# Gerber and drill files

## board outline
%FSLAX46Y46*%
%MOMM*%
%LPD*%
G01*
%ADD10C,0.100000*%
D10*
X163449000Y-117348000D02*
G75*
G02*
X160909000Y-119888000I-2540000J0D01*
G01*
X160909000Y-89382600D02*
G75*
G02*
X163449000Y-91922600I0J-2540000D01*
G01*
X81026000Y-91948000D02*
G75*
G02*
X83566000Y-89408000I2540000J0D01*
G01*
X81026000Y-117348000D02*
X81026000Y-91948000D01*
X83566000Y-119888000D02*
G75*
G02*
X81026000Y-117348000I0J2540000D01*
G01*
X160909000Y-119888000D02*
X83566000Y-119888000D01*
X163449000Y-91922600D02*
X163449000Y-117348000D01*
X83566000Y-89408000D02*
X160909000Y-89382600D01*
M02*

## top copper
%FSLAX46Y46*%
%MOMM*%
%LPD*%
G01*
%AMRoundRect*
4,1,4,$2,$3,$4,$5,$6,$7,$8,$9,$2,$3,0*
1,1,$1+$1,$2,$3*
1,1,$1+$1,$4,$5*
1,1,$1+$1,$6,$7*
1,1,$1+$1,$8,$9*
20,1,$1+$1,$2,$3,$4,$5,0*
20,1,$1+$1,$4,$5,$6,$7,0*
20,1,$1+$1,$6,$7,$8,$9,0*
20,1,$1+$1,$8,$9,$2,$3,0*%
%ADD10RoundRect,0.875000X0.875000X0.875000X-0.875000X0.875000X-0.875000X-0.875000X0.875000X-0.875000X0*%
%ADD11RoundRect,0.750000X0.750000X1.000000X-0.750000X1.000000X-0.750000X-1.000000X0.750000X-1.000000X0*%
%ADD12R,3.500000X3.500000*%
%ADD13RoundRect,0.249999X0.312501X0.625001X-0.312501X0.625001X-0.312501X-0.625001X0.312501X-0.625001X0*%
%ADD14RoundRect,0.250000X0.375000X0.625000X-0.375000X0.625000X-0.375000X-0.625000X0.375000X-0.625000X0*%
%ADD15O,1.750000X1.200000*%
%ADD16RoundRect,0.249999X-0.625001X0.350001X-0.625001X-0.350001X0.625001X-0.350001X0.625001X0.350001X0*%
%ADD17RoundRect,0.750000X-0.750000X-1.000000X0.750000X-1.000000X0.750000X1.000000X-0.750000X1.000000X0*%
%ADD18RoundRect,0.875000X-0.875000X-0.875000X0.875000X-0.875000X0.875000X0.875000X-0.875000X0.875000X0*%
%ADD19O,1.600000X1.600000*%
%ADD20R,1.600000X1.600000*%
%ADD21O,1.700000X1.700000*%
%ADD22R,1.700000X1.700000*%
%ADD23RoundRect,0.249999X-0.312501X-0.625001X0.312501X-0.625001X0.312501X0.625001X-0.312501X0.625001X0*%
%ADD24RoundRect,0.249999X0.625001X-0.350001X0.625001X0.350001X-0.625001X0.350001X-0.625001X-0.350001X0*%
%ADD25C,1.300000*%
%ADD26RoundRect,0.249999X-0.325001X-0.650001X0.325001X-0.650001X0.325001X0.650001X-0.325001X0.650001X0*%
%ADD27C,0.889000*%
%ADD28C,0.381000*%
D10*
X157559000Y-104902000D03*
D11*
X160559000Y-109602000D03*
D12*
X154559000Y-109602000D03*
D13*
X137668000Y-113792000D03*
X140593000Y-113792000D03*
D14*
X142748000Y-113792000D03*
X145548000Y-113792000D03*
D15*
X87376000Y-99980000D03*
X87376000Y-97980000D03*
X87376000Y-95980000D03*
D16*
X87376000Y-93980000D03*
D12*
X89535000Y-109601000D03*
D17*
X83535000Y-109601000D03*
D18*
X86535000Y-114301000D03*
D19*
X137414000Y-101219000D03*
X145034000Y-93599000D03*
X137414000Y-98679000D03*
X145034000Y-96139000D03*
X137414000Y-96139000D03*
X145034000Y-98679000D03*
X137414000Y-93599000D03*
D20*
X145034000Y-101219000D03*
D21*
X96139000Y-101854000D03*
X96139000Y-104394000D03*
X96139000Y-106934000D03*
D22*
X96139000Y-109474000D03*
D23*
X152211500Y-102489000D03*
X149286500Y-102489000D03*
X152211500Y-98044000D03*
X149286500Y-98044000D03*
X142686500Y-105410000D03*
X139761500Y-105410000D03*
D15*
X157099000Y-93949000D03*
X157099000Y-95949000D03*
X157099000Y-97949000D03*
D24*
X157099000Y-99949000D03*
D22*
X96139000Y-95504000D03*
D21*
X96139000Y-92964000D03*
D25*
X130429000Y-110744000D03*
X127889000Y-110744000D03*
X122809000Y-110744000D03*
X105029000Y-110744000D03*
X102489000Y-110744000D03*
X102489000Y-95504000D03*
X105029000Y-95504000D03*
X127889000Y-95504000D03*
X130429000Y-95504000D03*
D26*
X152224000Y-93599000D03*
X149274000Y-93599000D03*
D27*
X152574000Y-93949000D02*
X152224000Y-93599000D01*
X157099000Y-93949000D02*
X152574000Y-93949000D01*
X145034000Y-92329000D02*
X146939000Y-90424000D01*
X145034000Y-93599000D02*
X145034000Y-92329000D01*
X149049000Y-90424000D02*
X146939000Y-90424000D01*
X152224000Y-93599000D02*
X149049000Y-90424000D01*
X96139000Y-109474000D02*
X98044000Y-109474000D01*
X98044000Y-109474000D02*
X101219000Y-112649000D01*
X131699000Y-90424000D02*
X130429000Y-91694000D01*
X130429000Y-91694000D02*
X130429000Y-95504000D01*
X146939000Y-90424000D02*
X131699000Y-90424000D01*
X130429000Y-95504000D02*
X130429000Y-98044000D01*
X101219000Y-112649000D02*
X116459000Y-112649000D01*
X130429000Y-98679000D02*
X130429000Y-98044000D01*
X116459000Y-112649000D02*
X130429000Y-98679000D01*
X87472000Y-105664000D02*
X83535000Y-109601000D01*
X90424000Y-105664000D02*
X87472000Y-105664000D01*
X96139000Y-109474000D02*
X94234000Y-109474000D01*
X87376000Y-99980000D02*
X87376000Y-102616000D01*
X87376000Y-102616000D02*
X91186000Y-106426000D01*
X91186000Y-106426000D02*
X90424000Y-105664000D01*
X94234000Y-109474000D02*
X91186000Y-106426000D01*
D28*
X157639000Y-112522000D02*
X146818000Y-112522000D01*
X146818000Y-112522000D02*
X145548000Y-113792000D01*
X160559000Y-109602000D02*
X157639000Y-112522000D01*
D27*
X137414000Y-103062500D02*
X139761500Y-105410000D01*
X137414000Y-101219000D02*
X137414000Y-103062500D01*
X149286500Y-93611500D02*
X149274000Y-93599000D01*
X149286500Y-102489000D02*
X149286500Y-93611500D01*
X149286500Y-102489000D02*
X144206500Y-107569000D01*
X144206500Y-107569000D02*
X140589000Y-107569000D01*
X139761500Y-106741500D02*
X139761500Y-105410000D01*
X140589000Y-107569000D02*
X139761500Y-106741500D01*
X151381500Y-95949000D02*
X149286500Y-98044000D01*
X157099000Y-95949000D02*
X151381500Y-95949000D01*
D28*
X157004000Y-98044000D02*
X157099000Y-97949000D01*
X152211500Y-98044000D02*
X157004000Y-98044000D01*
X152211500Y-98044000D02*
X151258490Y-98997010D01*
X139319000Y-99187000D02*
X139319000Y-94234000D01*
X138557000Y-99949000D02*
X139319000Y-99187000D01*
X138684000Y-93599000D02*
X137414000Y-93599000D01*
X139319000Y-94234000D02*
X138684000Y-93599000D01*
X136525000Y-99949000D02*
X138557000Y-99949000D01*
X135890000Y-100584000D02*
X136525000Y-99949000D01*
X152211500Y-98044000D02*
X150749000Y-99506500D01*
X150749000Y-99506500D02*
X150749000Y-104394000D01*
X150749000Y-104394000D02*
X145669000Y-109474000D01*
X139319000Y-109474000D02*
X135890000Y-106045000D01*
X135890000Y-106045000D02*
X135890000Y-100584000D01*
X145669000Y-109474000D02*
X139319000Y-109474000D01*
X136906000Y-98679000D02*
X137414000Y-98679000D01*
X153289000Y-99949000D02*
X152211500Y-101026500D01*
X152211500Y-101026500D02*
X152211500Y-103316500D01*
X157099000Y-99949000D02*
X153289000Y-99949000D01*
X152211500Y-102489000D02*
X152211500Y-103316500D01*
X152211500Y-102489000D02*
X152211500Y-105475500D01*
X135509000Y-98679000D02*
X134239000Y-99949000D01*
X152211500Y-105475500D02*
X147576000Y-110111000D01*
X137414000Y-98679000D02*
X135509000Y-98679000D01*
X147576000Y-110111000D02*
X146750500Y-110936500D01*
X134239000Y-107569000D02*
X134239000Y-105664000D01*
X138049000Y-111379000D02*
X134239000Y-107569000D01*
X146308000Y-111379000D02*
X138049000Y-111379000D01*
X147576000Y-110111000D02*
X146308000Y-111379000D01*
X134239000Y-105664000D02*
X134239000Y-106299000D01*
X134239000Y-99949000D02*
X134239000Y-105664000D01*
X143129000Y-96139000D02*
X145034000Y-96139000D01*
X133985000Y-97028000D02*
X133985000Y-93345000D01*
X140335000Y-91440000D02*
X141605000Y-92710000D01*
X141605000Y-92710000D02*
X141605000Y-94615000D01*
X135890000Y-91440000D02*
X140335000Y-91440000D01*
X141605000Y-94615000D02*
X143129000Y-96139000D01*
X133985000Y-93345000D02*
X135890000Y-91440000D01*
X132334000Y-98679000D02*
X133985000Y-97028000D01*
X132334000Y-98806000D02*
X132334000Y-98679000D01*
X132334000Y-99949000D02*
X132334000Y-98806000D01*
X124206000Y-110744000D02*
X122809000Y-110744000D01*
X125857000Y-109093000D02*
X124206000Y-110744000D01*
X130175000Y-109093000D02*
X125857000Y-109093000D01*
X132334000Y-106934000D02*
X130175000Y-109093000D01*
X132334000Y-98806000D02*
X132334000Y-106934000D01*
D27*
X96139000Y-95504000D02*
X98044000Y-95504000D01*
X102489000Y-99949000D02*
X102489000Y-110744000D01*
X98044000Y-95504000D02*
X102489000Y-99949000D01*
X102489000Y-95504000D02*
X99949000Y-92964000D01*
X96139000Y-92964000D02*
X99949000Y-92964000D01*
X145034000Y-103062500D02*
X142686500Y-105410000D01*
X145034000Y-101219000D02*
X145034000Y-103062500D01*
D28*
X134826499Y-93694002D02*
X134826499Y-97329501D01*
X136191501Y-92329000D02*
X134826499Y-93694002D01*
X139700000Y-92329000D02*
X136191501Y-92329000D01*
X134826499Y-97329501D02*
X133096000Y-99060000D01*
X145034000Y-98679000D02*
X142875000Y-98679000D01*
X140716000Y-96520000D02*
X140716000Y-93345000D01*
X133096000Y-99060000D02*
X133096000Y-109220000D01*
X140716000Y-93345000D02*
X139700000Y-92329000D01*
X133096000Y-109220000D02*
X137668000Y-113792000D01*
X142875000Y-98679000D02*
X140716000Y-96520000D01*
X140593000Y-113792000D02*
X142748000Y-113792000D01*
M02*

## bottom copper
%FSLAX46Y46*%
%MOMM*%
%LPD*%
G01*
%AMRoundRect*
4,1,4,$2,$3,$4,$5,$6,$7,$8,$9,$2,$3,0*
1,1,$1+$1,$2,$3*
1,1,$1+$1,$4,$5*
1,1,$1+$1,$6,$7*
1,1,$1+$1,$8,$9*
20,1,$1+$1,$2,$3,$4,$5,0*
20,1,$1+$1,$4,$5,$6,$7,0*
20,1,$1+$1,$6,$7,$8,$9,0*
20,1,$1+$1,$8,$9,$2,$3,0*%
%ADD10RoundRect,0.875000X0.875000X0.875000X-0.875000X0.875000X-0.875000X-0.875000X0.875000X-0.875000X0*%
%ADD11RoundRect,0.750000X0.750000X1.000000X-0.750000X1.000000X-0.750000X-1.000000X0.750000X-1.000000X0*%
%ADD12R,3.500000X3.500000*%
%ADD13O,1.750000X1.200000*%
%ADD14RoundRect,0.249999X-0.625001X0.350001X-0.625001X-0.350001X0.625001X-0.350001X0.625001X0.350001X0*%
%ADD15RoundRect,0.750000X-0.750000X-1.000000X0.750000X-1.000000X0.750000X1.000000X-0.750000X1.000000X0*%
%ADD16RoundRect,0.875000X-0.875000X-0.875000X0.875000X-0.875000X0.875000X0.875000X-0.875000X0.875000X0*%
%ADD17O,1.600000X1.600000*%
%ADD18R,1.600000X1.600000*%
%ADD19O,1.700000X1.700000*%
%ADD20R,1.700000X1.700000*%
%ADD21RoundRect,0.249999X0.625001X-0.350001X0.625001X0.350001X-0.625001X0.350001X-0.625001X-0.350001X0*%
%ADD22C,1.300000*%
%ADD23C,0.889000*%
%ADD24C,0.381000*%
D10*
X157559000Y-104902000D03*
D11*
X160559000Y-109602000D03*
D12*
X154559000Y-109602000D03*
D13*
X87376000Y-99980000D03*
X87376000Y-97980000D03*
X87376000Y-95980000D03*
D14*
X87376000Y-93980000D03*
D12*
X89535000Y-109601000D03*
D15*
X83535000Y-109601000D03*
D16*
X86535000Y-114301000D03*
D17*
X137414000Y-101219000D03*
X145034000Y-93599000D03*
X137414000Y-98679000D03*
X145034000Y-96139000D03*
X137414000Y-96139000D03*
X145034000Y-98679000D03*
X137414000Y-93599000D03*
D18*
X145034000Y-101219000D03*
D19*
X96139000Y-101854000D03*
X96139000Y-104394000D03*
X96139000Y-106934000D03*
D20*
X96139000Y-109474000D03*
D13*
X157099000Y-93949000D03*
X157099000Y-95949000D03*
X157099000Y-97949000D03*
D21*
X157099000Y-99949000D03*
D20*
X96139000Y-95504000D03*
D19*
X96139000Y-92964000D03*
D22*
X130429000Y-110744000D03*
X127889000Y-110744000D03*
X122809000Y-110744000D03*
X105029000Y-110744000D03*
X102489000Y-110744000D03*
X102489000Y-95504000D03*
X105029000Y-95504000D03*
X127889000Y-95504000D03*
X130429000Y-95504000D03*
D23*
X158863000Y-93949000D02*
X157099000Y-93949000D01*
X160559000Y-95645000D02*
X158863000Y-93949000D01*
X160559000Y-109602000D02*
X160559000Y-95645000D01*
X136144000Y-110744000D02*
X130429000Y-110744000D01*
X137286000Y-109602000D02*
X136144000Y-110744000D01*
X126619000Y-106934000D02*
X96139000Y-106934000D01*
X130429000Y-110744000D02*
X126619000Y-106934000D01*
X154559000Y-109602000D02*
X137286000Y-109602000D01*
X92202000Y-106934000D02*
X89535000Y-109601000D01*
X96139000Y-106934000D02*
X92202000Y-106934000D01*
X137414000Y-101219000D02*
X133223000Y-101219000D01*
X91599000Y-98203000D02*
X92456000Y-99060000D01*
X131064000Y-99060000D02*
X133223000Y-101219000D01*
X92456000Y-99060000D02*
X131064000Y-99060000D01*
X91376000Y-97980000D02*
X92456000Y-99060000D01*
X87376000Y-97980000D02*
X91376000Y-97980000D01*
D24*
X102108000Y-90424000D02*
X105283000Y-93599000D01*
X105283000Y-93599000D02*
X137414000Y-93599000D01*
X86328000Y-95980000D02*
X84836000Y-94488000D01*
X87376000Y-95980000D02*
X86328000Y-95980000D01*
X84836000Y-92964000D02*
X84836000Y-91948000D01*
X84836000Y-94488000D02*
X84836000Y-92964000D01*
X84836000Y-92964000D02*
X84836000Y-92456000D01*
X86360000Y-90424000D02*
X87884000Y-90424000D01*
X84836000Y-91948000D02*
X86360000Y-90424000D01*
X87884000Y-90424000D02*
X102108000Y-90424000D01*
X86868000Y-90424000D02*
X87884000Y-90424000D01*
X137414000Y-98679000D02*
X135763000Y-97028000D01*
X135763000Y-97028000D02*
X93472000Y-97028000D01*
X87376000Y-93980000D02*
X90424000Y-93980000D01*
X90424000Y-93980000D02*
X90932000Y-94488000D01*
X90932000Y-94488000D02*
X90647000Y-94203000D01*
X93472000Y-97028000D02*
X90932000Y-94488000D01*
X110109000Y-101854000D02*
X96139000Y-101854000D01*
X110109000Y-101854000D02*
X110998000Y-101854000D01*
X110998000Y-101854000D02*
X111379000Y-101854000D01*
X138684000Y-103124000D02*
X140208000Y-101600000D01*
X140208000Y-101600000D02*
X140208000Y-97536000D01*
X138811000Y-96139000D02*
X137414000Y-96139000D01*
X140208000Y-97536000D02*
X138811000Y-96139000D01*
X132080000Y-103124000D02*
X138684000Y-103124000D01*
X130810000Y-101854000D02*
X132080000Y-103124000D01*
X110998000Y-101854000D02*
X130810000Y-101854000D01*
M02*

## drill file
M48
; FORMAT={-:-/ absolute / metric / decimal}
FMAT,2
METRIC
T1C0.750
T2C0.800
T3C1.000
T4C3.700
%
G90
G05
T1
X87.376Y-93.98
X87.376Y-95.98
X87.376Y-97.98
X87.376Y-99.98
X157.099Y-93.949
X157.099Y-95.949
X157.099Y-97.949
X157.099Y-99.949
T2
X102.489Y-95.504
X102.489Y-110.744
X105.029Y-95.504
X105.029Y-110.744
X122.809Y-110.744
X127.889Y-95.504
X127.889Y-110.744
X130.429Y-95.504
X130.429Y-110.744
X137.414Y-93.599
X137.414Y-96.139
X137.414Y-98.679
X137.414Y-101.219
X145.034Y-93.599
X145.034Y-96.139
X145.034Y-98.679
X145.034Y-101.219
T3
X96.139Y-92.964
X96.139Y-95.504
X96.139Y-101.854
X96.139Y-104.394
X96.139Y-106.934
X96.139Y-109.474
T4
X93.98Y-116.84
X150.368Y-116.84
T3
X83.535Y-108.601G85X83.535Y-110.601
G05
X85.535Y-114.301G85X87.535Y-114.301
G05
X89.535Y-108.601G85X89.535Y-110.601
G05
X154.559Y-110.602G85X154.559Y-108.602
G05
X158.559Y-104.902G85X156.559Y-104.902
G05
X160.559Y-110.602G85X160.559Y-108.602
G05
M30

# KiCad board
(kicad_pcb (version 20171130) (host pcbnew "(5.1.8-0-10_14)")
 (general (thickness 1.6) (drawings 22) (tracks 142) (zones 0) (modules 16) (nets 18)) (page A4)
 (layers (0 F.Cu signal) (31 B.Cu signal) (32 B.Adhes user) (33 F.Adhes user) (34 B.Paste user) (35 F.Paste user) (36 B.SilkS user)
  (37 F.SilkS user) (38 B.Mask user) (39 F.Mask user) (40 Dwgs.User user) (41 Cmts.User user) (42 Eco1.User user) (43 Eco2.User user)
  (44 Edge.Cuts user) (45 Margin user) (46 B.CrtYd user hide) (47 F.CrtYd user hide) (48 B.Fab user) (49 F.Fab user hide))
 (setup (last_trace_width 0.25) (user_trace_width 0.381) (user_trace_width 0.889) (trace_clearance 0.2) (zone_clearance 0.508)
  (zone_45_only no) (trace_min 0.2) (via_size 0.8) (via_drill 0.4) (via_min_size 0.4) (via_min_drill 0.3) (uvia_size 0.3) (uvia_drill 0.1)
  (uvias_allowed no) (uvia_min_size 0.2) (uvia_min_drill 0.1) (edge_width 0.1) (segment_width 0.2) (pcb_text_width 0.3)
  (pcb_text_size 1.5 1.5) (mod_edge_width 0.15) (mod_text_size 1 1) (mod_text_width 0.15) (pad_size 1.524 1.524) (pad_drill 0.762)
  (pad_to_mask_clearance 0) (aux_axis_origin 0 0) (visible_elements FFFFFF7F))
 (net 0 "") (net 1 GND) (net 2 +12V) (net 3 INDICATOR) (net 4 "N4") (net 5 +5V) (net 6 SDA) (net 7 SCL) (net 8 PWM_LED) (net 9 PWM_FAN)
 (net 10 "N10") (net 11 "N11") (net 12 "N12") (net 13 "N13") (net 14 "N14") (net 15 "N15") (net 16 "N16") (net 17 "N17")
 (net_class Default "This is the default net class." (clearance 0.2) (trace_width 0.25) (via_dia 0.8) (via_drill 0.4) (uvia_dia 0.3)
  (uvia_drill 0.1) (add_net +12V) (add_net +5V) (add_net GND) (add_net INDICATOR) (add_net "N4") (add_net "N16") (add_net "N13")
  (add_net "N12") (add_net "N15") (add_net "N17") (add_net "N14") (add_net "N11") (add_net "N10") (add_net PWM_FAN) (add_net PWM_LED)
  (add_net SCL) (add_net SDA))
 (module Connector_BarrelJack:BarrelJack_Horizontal (layer F.Cu) (at 154.559 109.602 180)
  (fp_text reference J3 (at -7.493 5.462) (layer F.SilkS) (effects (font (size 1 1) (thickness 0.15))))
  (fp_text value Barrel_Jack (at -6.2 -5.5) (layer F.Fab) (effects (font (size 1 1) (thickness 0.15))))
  (pad 3 thru_hole roundrect (at -3 4.7 180) (size 3.5 3.5) (drill oval 3 1) (layers *.Cu *.Mask) (roundrect_rratio 0.25))
  (pad 2 thru_hole roundrect (at -6 0 180) (size 3 3.5) (drill oval 1 3) (layers *.Cu *.Mask) (roundrect_rratio 0.25) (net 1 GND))
  (pad 1 thru_hole rect (at 0 0 180) (size 3.5 3.5) (drill oval 1 3) (layers *.Cu *.Mask) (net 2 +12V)))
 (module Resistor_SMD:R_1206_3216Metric (layer F.Cu) (at 139.1305 113.792 180)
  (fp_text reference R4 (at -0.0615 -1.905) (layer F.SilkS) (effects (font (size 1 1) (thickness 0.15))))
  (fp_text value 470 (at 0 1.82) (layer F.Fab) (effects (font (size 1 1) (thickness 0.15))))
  (pad 2 smd roundrect (at 1.4625 0 180) (size 1.125 1.75) (layers F.Cu F.Paste F.Mask) (roundrect_rratio 0.2222213333333333)
   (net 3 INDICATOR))
  (pad 1 smd roundrect (at -1.4625 0 180) (size 1.125 1.75) (layers F.Cu F.Paste F.Mask) (roundrect_rratio 0.2222213333333333) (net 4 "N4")))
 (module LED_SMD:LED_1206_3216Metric (layer F.Cu) (at 144.148 113.792 180)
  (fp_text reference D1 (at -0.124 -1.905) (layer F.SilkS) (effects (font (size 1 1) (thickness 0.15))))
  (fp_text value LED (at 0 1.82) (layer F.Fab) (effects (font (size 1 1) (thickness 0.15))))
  (pad 2 smd roundrect (at 1.4 0 180) (size 1.25 1.75) (layers F.Cu F.Paste F.Mask) (roundrect_rratio 0.2) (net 4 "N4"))
  (pad 1 smd roundrect (at -1.4 0 180) (size 1.25 1.75) (layers F.Cu F.Paste F.Mask) (roundrect_rratio 0.2) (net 1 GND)))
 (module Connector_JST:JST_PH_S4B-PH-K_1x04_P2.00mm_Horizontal (layer F.Cu) (at 87.376 93.98 270)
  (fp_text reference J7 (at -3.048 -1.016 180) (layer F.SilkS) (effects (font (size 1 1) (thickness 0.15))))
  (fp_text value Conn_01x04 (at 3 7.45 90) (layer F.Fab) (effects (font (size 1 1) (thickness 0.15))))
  (pad 4 thru_hole oval (at 6 0 270) (size 1.2 1.75) (drill 0.75) (layers *.Cu *.Mask) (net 1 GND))
  (pad 3 thru_hole oval (at 4 0 270) (size 1.2 1.75) (drill 0.75) (layers *.Cu *.Mask) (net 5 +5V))
  (pad 2 thru_hole oval (at 2 0 270) (size 1.2 1.75) (drill 0.75) (layers *.Cu *.Mask) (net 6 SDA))
  (pad 1 thru_hole roundrect (at 0 0 270) (size 1.2 1.75) (drill 0.75) (layers *.Cu *.Mask) (roundrect_rratio 0.2083325) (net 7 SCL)))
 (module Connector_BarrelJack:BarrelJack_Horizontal (layer F.Cu) (at 89.535 109.601)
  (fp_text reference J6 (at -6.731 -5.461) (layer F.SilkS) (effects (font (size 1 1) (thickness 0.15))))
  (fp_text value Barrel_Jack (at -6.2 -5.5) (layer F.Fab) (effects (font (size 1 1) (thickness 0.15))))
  (pad 1 thru_hole rect (at 0 0) (size 3.5 3.5) (drill oval 1 3) (layers *.Cu *.Mask) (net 2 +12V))
  (pad 2 thru_hole roundrect (at -6 0) (size 3 3.5) (drill oval 1 3) (layers *.Cu *.Mask) (roundrect_rratio 0.25) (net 1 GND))
  (pad 3 thru_hole roundrect (at -3 4.7) (size 3.5 3.5) (drill oval 3 1) (layers *.Cu *.Mask) (roundrect_rratio 0.25)))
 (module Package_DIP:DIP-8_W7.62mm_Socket (layer F.Cu) (at 145.034 101.219 180)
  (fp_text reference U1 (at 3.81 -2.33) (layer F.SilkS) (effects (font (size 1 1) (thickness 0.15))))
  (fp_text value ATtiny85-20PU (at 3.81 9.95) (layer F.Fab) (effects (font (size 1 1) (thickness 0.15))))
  (pad 8 thru_hole oval (at 7.62 0 180) (size 1.6 1.6) (drill 0.8) (layers *.Cu *.Mask) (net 5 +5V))
  (pad 4 thru_hole oval (at 0 7.62 180) (size 1.6 1.6) (drill 0.8) (layers *.Cu *.Mask) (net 1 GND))
  (pad 7 thru_hole oval (at 7.62 2.54 180) (size 1.6 1.6) (drill 0.8) (layers *.Cu *.Mask) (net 7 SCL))
  (pad 3 thru_hole oval (at 0 5.08 180) (size 1.6 1.6) (drill 0.8) (layers *.Cu *.Mask) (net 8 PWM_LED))
  (pad 6 thru_hole oval (at 7.62 5.08 180) (size 1.6 1.6) (drill 0.8) (layers *.Cu *.Mask) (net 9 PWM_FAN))
  (pad 2 thru_hole oval (at 0 2.54 180) (size 1.6 1.6) (drill 0.8) (layers *.Cu *.Mask) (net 3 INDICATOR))
  (pad 5 thru_hole oval (at 7.62 7.62 180) (size 1.6 1.6) (drill 0.8) (layers *.Cu *.Mask) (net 6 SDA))
  (pad 1 thru_hole rect (at 0 0 180) (size 1.6 1.6) (drill 0.8) (layers *.Cu *.Mask) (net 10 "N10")))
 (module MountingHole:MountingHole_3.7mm (layer F.Cu) (at 150.368 116.84 180)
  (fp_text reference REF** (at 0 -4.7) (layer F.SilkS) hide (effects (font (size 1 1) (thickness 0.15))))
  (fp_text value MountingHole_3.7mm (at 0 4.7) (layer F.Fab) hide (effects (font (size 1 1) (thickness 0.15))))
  (pad 1 np_thru_hole circle (at 0 0 180) (size 3.7 3.7) (drill 3.7) (layers *.Cu *.Mask)))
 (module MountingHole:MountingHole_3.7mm (layer F.Cu) (at 93.98 116.84 180)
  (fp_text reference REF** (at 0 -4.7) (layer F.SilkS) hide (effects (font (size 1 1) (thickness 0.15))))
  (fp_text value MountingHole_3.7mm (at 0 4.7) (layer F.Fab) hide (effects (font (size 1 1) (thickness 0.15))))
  (pad 1 np_thru_hole circle (at 0 0 180) (size 3.7 3.7) (drill 3.7) (layers *.Cu *.Mask)))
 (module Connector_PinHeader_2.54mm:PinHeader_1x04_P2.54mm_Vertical (layer F.Cu) (at 96.139 109.474 180)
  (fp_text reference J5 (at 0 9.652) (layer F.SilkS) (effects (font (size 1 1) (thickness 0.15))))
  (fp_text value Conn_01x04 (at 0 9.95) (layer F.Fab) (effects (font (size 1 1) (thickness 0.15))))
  (pad 4 thru_hole oval (at 0 7.62 180) (size 1.7 1.7) (drill 1) (layers *.Cu *.Mask) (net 9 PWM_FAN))
  (pad 3 thru_hole oval (at 0 5.08 180) (size 1.7 1.7) (drill 1) (layers *.Cu *.Mask) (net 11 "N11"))
  (pad 2 thru_hole oval (at 0 2.54 180) (size 1.7 1.7) (drill 1) (layers *.Cu *.Mask) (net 2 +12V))
  (pad 1 thru_hole rect (at 0 0 180) (size 1.7 1.7) (drill 1) (layers *.Cu *.Mask) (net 1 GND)))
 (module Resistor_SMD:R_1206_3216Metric (layer F.Cu) (at 150.749 102.489)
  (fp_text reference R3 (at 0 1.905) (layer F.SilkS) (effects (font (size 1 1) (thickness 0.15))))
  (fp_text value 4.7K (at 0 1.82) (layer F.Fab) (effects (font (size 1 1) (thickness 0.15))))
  (pad 2 smd roundrect (at 1.4625 0) (size 1.125 1.75) (layers F.Cu F.Paste F.Mask) (roundrect_rratio 0.2222213333333333) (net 7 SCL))
  (pad 1 smd roundrect (at -1.4625 0) (size 1.125 1.75) (layers F.Cu F.Paste F.Mask) (roundrect_rratio 0.2222213333333333) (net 5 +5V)))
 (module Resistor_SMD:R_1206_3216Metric (layer F.Cu) (at 150.749 98.044)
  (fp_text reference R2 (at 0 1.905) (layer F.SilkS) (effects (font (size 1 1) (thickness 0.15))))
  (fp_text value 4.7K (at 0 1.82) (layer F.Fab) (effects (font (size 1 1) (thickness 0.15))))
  (pad 2 smd roundrect (at 1.4625 0) (size 1.125 1.75) (layers F.Cu F.Paste F.Mask) (roundrect_rratio 0.2222213333333333) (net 6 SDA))
  (pad 1 smd roundrect (at -1.4625 0) (size 1.125 1.75) (layers F.Cu F.Paste F.Mask) (roundrect_rratio 0.2222213333333333) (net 5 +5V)))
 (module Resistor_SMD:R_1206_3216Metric (layer F.Cu) (at 141.224 105.41)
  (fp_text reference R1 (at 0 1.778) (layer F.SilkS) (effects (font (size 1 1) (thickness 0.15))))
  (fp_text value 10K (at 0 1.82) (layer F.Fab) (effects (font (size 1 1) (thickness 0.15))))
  (pad 2 smd roundrect (at 1.4625 0) (size 1.125 1.75) (layers F.Cu F.Paste F.Mask) (roundrect_rratio 0.2222213333333333) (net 10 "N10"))
  (pad 1 smd roundrect (at -1.4625 0) (size 1.125 1.75) (layers F.Cu F.Paste F.Mask) (roundrect_rratio 0.2222213333333333) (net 5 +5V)))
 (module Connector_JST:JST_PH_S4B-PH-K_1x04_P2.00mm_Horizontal (layer F.Cu) (at 157.099 99.949 90)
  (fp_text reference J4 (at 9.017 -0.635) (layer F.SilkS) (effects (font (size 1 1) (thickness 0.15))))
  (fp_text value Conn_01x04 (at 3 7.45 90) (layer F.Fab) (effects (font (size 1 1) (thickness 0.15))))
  (pad 4 thru_hole oval (at 6 0 90) (size 1.2 1.75) (drill 0.75) (layers *.Cu *.Mask) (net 1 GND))
  (pad 3 thru_hole oval (at 4 0 90) (size 1.2 1.75) (drill 0.75) (layers *.Cu *.Mask) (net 5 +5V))
  (pad 2 thru_hole oval (at 2 0 90) (size 1.2 1.75) (drill 0.75) (layers *.Cu *.Mask) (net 6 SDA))
  (pad 1 thru_hole roundrect (at 0 0 90) (size 1.2 1.75) (drill 0.75) (layers *.Cu *.Mask) (roundrect_rratio 0.2083325) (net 7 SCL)))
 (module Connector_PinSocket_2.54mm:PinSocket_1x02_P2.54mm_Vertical (layer F.Cu) (at 96.139 95.504 180)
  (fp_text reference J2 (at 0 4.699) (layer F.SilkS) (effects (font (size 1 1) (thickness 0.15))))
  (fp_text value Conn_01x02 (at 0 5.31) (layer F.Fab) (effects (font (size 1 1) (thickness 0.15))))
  (pad 1 thru_hole rect (at 0 0 180) (size 1.7 1.7) (drill 1) (layers *.Cu *.Mask) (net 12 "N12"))
  (pad 2 thru_hole oval (at 0 2.54 180) (size 1.7 1.7) (drill 1) (layers *.Cu *.Mask) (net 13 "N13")))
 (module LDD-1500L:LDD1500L (layer F.Cu) (at 130.429 95.504 270)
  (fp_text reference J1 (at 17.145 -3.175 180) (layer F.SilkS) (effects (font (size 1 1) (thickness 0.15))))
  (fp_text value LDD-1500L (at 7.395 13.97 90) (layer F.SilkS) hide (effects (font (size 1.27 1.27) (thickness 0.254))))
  (pad 24 thru_hole circle (at 15.24 0) (size 1.3 1.3) (drill 0.8) (layers *.Cu *.Mask F.SilkS) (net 2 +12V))
  (pad 23 thru_hole circle (at 15.24 2.54) (size 1.3 1.3) (drill 0.8) (layers *.Cu *.Mask F.SilkS) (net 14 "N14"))
  (pad 21 thru_hole circle (at 15.24 7.62) (size 1.3 1.3) (drill 0.8) (layers *.Cu *.Mask F.SilkS) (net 8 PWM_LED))
  (pad 14 thru_hole circle (at 15.24 25.4) (size 1.3 1.3) (drill 0.8) (layers *.Cu *.Mask F.SilkS) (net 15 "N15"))
  (pad 13 thru_hole circle (at 15.24 27.94) (size 1.3 1.3) (drill 0.8) (layers *.Cu *.Mask F.SilkS) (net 12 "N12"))
  (pad 12 thru_hole circle (at 0 27.94) (size 1.3 1.3) (drill 0.8) (layers *.Cu *.Mask F.SilkS) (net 13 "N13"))
  (pad 11 thru_hole circle (at 0 25.4) (size 1.3 1.3) (drill 0.8) (layers *.Cu *.Mask F.SilkS) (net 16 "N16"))
  (pad 2 thru_hole circle (at 0 2.54) (size 1.3 1.3) (drill 0.8) (layers *.Cu *.Mask F.SilkS) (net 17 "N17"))
  (pad 1 thru_hole circle (at 0 0) (size 1.3 1.3) (drill 0.8) (layers *.Cu *.Mask F.SilkS) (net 1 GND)))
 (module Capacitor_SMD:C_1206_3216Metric (layer F.Cu) (at 150.749 93.599)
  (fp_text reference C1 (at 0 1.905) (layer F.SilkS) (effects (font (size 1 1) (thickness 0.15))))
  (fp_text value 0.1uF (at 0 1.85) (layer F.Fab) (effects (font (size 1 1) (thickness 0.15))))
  (pad 2 smd roundrect (at 1.475 0) (size 1.15 1.8) (layers F.Cu F.Paste F.Mask) (roundrect_rratio 0.2173904347826087) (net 1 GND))
  (pad 1 smd roundrect (at -1.475 0) (size 1.15 1.8) (layers F.Cu F.Paste F.Mask) (roundrect_rratio 0.2173904347826087) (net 5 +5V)))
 (gr_arc (start 160.909 117.348) (end 160.909 119.888) (angle -90) (layer Edge.Cuts) (width 0.1))
 (gr_arc (start 160.909 91.9226) (end 163.449 91.9226) (angle -90) (layer Edge.Cuts) (width 0.1))
 (gr_arc (start 83.566 91.948) (end 83.566 89.408) (angle -90) (layer Edge.Cuts) (width 0.1))
 (gr_line (start 81.026 117.348) (end 81.026 91.948) (layer Edge.Cuts) (width 0.1))
 (gr_arc (start 83.566 117.348) (end 81.026 117.348) (angle -90) (layer Edge.Cuts) (width 0.1))
 (gr_line (start 160.909 119.888) (end 83.566 119.888) (layer Edge.Cuts) (width 0.1))
 (gr_line (start 163.449 91.9226) (end 163.449 117.348) (layer Edge.Cuts) (width 0.1))
 (gr_line (start 83.566 89.408) (end 160.909 89.3826) (layer Edge.Cuts) (width 0.1))
 (segment (start 152.574 93.949) (end 152.224 93.599) (width 0.889) (layer F.Cu) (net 1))
 (segment (start 157.099 93.949) (end 152.574 93.949) (width 0.889) (layer F.Cu) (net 1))
 (segment (start 158.863 93.949) (end 157.099 93.949) (width 0.889) (layer B.Cu) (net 1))
 (segment (start 160.559 95.645) (end 158.863 93.949) (width 0.889) (layer B.Cu) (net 1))
 (segment (start 160.559 109.602) (end 160.559 95.645) (width 0.889) (layer B.Cu) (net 1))
 (segment (start 145.034 92.329) (end 146.939 90.424) (width 0.889) (layer F.Cu) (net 1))
 (segment (start 145.034 93.599) (end 145.034 92.329) (width 0.889) (layer F.Cu) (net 1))
 (segment (start 149.049 90.424) (end 146.939 90.424) (width 0.889) (layer F.Cu) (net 1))
 (segment (start 152.224 93.599) (end 149.049 90.424) (width 0.889) (layer F.Cu) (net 1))
 (segment (start 96.139 109.474) (end 98.044 109.474) (width 0.889) (layer F.Cu) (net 1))
 (segment (start 98.044 109.474) (end 101.219 112.649) (width 0.889) (layer F.Cu) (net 1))
 (segment (start 131.699 90.424) (end 130.429 91.694) (width 0.889) (layer F.Cu) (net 1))
 (segment (start 130.429 91.694) (end 130.429 95.504) (width 0.889) (layer F.Cu) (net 1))
 (segment (start 146.939 90.424) (end 131.699 90.424) (width 0.889) (layer F.Cu) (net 1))
 (segment (start 130.429 95.504) (end 130.429 98.044) (width 0.889) (layer F.Cu) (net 1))
 (segment (start 101.219 112.649) (end 116.459 112.649) (width 0.889) (layer F.Cu) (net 1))
 (segment (start 130.429 98.679) (end 130.429 98.044) (width 0.889) (layer F.Cu) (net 1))
 (segment (start 116.459 112.649) (end 130.429 98.679) (width 0.889) (layer F.Cu) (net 1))
 (segment (start 87.472 105.664) (end 83.535 109.601) (width 0.889) (layer F.Cu) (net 1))
 (segment (start 90.424 105.664) (end 87.472 105.664) (width 0.889) (layer F.Cu) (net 1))
 (segment (start 96.139 109.474) (end 94.234 109.474) (width 0.889) (layer F.Cu) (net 1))
 (segment (start 87.376 99.98) (end 87.376 102.616) (width 0.889) (layer F.Cu) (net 1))
 (segment (start 87.376 102.616) (end 91.186 106.426) (width 0.889) (layer F.Cu) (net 1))
 (segment (start 91.186 106.426) (end 90.424 105.664) (width 0.889) (layer F.Cu) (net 1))
 (segment (start 94.234 109.474) (end 91.186 106.426) (width 0.889) (layer F.Cu) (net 1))
 (segment (start 157.639 112.522) (end 146.818 112.522) (width 0.381) (layer F.Cu) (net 1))
 (segment (start 146.818 112.522) (end 145.548 113.792) (width 0.381) (layer F.Cu) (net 1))
 (segment (start 160.559 109.602) (end 157.639 112.522) (width 0.381) (layer F.Cu) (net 1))
 (segment (start 136.144 110.744) (end 130.429 110.744) (width 0.889) (layer B.Cu) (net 2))
 (segment (start 137.286 109.602) (end 136.144 110.744) (width 0.889) (layer B.Cu) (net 2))
 (segment (start 126.619 106.934) (end 96.139 106.934) (width 0.889) (layer B.Cu) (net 2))
 (segment (start 130.429 110.744) (end 126.619 106.934) (width 0.889) (layer B.Cu) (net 2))
 (segment (start 154.559 109.602) (end 137.286 109.602) (width 0.889) (layer B.Cu) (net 2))
 (segment (start 92.202 106.934) (end 89.535 109.601) (width 0.889) (layer B.Cu) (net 2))
 (segment (start 96.139 106.934) (end 92.202 106.934) (width 0.889) (layer B.Cu) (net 2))
 (segment (start 137.414 103.0625) (end 139.7615 105.41) (width 0.889) (layer F.Cu) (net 5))
 (segment (start 137.414 101.219) (end 137.414 103.0625) (width 0.889) (layer F.Cu) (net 5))
 (segment (start 149.2865 93.6115) (end 149.274 93.599) (width 0.889) (layer F.Cu) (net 5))
 (segment (start 149.2865 102.489) (end 149.2865 93.6115) (width 0.889) (layer F.Cu) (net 5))
 (segment (start 149.2865 102.489) (end 144.2065 107.569) (width 0.889) (layer F.Cu) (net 5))
 (segment (start 144.2065 107.569) (end 140.589 107.569) (width 0.889) (layer F.Cu) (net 5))
 (segment (start 139.7615 106.7415) (end 139.7615 105.41) (width 0.889) (layer F.Cu) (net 5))
 (segment (start 140.589 107.569) (end 139.7615 106.7415) (width 0.889) (layer F.Cu) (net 5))
 (segment (start 151.3815 95.949) (end 149.2865 98.044) (width 0.889) (layer F.Cu) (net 5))
 (segment (start 157.099 95.949) (end 151.3815 95.949) (width 0.889) (layer F.Cu) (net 5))
 (segment (start 137.414 101.219) (end 133.223 101.219) (width 0.889) (layer B.Cu) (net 5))
 (segment (start 91.599 98.203) (end 92.456 99.06) (width 0.889) (layer B.Cu) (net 5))
 (segment (start 131.064 99.06) (end 133.223 101.219) (width 0.889) (layer B.Cu) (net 5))
 (segment (start 92.456 99.06) (end 131.064 99.06) (width 0.889) (layer B.Cu) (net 5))
 (segment (start 91.376 97.98) (end 92.456 99.06) (width 0.889) (layer B.Cu) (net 5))
 (segment (start 87.376 97.98) (end 91.376 97.98) (width 0.889) (layer B.Cu) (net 5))
 (segment (start 157.004 98.044) (end 157.099 97.949) (width 0.381) (layer F.Cu) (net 6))
 (segment (start 152.2115 98.044) (end 157.004 98.044) (width 0.381) (layer F.Cu) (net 6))
 (segment (start 152.2115 98.044) (end 151.25849 98.99701) (width 0.381) (layer F.Cu) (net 6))
 (segment (start 139.319 99.187) (end 139.319 94.234) (width 0.381) (layer F.Cu) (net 6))
 (segment (start 138.557 99.949) (end 139.319 99.187) (width 0.381) (layer F.Cu) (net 6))
 (segment (start 138.684 93.599) (end 137.414 93.599) (width 0.381) (layer F.Cu) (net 6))
 (segment (start 139.319 94.234) (end 138.684 93.599) (width 0.381) (layer F.Cu) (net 6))
 (segment (start 136.525 99.949) (end 138.557 99.949) (width 0.381) (layer F.Cu) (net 6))
 (segment (start 135.89 100.584) (end 136.525 99.949) (width 0.381) (layer F.Cu) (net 6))
 (segment (start 152.2115 98.044) (end 150.749 99.5065) (width 0.381) (layer F.Cu) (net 6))
 (segment (start 150.749 99.5065) (end 150.749 104.394) (width 0.381) (layer F.Cu) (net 6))
 (segment (start 150.749 104.394) (end 145.669 109.474) (width 0.381) (layer F.Cu) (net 6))
 (segment (start 139.319 109.474) (end 135.89 106.045) (width 0.381) (layer F.Cu) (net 6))
 (segment (start 135.89 106.045) (end 135.89 100.584) (width 0.381) (layer F.Cu) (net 6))
 (segment (start 145.669 109.474) (end 139.319 109.474) (width 0.381) (layer F.Cu) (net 6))
 (segment (start 102.108 90.424) (end 105.283 93.599) (width 0.381) (layer B.Cu) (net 6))
 (segment (start 105.283 93.599) (end 137.414 93.599) (width 0.381) (layer B.Cu) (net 6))
 (segment (start 86.328 95.98) (end 84.836 94.488) (width 0.381) (layer B.Cu) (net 6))
 (segment (start 87.376 95.98) (end 86.328 95.98) (width 0.381) (layer B.Cu) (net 6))
 (segment (start 84.836 92.964) (end 84.836 91.948) (width 0.381) (layer B.Cu) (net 6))
 (segment (start 84.836 94.488) (end 84.836 92.964) (width 0.381) (layer B.Cu) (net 6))
 (segment (start 84.836 92.964) (end 84.836 92.456) (width 0.381) (layer B.Cu) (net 6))
 (segment (start 86.36 90.424) (end 87.884 90.424) (width 0.381) (layer B.Cu) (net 6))
 (segment (start 84.836 91.948) (end 86.36 90.424) (width 0.381) (layer B.Cu) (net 6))
 (segment (start 87.884 90.424) (end 102.108 90.424) (width 0.381) (layer B.Cu) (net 6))
 (segment (start 86.868 90.424) (end 87.884 90.424) (width 0.381) (layer B.Cu) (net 6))
 (segment (start 136.906 98.679) (end 137.414 98.679) (width 0.381) (layer F.Cu) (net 7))
 (segment (start 153.289 99.949) (end 152.2115 101.0265) (width 0.381) (layer F.Cu) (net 7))
 (segment (start 152.2115 101.0265) (end 152.2115 103.3165) (width 0.381) (layer F.Cu) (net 7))
 (segment (start 157.099 99.949) (end 153.289 99.949) (width 0.381) (layer F.Cu) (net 7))
 (segment (start 152.2115 102.489) (end 152.2115 103.3165) (width 0.381) (layer F.Cu) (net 7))
 (segment (start 152.2115 102.489) (end 152.2115 105.4755) (width 0.381) (layer F.Cu) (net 7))
 (segment (start 135.509 98.679) (end 134.239 99.949) (width 0.381) (layer F.Cu) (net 7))
 (segment (start 152.2115 105.4755) (end 147.576 110.111) (width 0.381) (layer F.Cu) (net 7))
 (segment (start 137.414 98.679) (end 135.509 98.679) (width 0.381) (layer F.Cu) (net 7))
 (segment (start 147.576 110.111) (end 146.7505 110.9365) (width 0.381) (layer F.Cu) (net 7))
 (segment (start 134.239 107.569) (end 134.239 105.664) (width 0.381) (layer F.Cu) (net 7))
 (segment (start 138.049 111.379) (end 134.239 107.569) (width 0.381) (layer F.Cu) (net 7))
 (segment (start 146.308 111.379) (end 138.049 111.379) (width 0.381) (layer F.Cu) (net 7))
 (segment (start 147.576 110.111) (end 146.308 111.379) (width 0.381) (layer F.Cu) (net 7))
 (segment (start 134.239 105.664) (end 134.239 106.299) (width 0.381) (layer F.Cu) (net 7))
 (segment (start 134.239 99.949) (end 134.239 105.664) (width 0.381) (layer F.Cu) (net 7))
 (segment (start 137.414 98.679) (end 135.763 97.028) (width 0.381) (layer B.Cu) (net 7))
 (segment (start 135.763 97.028) (end 93.472 97.028) (width 0.381) (layer B.Cu) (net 7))
 (segment (start 87.376 93.98) (end 90.424 93.98) (width 0.381) (layer B.Cu) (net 7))
 (segment (start 90.424 93.98) (end 90.932 94.488) (width 0.381) (layer B.Cu) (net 7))
 (segment (start 90.932 94.488) (end 90.647 94.203) (width 0.381) (layer B.Cu) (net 7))
 (segment (start 93.472 97.028) (end 90.932 94.488) (width 0.381) (layer B.Cu) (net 7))
 (segment (start 143.129 96.139) (end 145.034 96.139) (width 0.381) (layer F.Cu) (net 8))
 (segment (start 133.985 97.028) (end 133.985 93.345) (width 0.381) (layer F.Cu) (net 8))
 (segment (start 140.335 91.44) (end 141.605 92.71) (width 0.381) (layer F.Cu) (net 8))
 (segment (start 141.605 92.71) (end 141.605 94.615) (width 0.381) (layer F.Cu) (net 8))
 (segment (start 135.89 91.44) (end 140.335 91.44) (width 0.381) (layer F.Cu) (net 8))
 (segment (start 141.605 94.615) (end 143.129 96.139) (width 0.381) (layer F.Cu) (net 8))
 (segment (start 133.985 93.345) (end 135.89 91.44) (width 0.381) (layer F.Cu) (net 8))
 (segment (start 132.334 98.679) (end 133.985 97.028) (width 0.381) (layer F.Cu) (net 8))
 (segment (start 132.334 98.806) (end 132.334 98.679) (width 0.381) (layer F.Cu) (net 8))
 (segment (start 132.334 99.949) (end 132.334 98.806) (width 0.381) (layer F.Cu) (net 8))
 (segment (start 124.206 110.744) (end 122.809 110.744) (width 0.381) (layer F.Cu) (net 8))
 (segment (start 125.857 109.093) (end 124.206 110.744) (width 0.381) (layer F.Cu) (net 8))
 (segment (start 130.175 109.093) (end 125.857 109.093) (width 0.381) (layer F.Cu) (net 8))
 (segment (start 132.334 106.934) (end 130.175 109.093) (width 0.381) (layer F.Cu) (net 8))
 (segment (start 132.334 98.806) (end 132.334 106.934) (width 0.381) (layer F.Cu) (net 8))
 (segment (start 110.109 101.854) (end 96.139 101.854) (width 0.381) (layer B.Cu) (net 9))
 (segment (start 110.109 101.854) (end 110.998 101.854) (width 0.381) (layer B.Cu) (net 9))
 (segment (start 110.998 101.854) (end 111.379 101.854) (width 0.381) (layer B.Cu) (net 9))
 (segment (start 138.684 103.124) (end 140.208 101.6) (width 0.381) (layer B.Cu) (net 9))
 (segment (start 140.208 101.6) (end 140.208 97.536) (width 0.381) (layer B.Cu) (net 9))
 (segment (start 138.811 96.139) (end 137.414 96.139) (width 0.381) (layer B.Cu) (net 9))
 (segment (start 140.208 97.536) (end 138.811 96.139) (width 0.381) (layer B.Cu) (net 9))
 (segment (start 132.08 103.124) (end 138.684 103.124) (width 0.381) (layer B.Cu) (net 9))
 (segment (start 130.81 101.854) (end 132.08 103.124) (width 0.381) (layer B.Cu) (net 9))
 (segment (start 110.998 101.854) (end 130.81 101.854) (width 0.381) (layer B.Cu) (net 9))
 (segment (start 96.139 95.504) (end 98.044 95.504) (width 0.889) (layer F.Cu) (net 12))
 (segment (start 102.489 99.949) (end 102.489 110.744) (width 0.889) (layer F.Cu) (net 12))
 (segment (start 98.044 95.504) (end 102.489 99.949) (width 0.889) (layer F.Cu) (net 12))
 (segment (start 102.489 95.504) (end 99.949 92.964) (width 0.889) (layer F.Cu) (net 13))
 (segment (start 96.139 92.964) (end 99.949 92.964) (width 0.889) (layer F.Cu) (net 13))
 (segment (start 145.034 103.0625) (end 142.6865 105.41) (width 0.889) (layer F.Cu) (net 10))
 (segment (start 145.034 101.219) (end 145.034 103.0625) (width 0.889) (layer F.Cu) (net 10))
 (segment (start 134.826499 93.694002) (end 134.826499 97.329501) (width 0.381) (layer F.Cu) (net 3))
 (segment (start 136.191501 92.329) (end 134.826499 93.694002) (width 0.381) (layer F.Cu) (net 3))
 (segment (start 139.7 92.329) (end 136.191501 92.329) (width 0.381) (layer F.Cu) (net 3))
 (segment (start 134.826499 97.329501) (end 133.096 99.06) (width 0.381) (layer F.Cu) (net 3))
 (segment (start 145.034 98.679) (end 142.875 98.679) (width 0.381) (layer F.Cu) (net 3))
 (segment (start 140.716 96.52) (end 140.716 93.345) (width 0.381) (layer F.Cu) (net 3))
 (segment (start 133.096 99.06) (end 133.096 109.22) (width 0.381) (layer F.Cu) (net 3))
 (segment (start 140.716 93.345) (end 139.7 92.329) (width 0.381) (layer F.Cu) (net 3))
 (segment (start 133.096 109.22) (end 137.668 113.792) (width 0.381) (layer F.Cu) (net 3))
 (segment (start 142.875 98.679) (end 140.716 96.52) (width 0.381) (layer F.Cu) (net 3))
 (segment (start 140.593 113.792) (end 142.748 113.792) (width 0.381) (layer F.Cu) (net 4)))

